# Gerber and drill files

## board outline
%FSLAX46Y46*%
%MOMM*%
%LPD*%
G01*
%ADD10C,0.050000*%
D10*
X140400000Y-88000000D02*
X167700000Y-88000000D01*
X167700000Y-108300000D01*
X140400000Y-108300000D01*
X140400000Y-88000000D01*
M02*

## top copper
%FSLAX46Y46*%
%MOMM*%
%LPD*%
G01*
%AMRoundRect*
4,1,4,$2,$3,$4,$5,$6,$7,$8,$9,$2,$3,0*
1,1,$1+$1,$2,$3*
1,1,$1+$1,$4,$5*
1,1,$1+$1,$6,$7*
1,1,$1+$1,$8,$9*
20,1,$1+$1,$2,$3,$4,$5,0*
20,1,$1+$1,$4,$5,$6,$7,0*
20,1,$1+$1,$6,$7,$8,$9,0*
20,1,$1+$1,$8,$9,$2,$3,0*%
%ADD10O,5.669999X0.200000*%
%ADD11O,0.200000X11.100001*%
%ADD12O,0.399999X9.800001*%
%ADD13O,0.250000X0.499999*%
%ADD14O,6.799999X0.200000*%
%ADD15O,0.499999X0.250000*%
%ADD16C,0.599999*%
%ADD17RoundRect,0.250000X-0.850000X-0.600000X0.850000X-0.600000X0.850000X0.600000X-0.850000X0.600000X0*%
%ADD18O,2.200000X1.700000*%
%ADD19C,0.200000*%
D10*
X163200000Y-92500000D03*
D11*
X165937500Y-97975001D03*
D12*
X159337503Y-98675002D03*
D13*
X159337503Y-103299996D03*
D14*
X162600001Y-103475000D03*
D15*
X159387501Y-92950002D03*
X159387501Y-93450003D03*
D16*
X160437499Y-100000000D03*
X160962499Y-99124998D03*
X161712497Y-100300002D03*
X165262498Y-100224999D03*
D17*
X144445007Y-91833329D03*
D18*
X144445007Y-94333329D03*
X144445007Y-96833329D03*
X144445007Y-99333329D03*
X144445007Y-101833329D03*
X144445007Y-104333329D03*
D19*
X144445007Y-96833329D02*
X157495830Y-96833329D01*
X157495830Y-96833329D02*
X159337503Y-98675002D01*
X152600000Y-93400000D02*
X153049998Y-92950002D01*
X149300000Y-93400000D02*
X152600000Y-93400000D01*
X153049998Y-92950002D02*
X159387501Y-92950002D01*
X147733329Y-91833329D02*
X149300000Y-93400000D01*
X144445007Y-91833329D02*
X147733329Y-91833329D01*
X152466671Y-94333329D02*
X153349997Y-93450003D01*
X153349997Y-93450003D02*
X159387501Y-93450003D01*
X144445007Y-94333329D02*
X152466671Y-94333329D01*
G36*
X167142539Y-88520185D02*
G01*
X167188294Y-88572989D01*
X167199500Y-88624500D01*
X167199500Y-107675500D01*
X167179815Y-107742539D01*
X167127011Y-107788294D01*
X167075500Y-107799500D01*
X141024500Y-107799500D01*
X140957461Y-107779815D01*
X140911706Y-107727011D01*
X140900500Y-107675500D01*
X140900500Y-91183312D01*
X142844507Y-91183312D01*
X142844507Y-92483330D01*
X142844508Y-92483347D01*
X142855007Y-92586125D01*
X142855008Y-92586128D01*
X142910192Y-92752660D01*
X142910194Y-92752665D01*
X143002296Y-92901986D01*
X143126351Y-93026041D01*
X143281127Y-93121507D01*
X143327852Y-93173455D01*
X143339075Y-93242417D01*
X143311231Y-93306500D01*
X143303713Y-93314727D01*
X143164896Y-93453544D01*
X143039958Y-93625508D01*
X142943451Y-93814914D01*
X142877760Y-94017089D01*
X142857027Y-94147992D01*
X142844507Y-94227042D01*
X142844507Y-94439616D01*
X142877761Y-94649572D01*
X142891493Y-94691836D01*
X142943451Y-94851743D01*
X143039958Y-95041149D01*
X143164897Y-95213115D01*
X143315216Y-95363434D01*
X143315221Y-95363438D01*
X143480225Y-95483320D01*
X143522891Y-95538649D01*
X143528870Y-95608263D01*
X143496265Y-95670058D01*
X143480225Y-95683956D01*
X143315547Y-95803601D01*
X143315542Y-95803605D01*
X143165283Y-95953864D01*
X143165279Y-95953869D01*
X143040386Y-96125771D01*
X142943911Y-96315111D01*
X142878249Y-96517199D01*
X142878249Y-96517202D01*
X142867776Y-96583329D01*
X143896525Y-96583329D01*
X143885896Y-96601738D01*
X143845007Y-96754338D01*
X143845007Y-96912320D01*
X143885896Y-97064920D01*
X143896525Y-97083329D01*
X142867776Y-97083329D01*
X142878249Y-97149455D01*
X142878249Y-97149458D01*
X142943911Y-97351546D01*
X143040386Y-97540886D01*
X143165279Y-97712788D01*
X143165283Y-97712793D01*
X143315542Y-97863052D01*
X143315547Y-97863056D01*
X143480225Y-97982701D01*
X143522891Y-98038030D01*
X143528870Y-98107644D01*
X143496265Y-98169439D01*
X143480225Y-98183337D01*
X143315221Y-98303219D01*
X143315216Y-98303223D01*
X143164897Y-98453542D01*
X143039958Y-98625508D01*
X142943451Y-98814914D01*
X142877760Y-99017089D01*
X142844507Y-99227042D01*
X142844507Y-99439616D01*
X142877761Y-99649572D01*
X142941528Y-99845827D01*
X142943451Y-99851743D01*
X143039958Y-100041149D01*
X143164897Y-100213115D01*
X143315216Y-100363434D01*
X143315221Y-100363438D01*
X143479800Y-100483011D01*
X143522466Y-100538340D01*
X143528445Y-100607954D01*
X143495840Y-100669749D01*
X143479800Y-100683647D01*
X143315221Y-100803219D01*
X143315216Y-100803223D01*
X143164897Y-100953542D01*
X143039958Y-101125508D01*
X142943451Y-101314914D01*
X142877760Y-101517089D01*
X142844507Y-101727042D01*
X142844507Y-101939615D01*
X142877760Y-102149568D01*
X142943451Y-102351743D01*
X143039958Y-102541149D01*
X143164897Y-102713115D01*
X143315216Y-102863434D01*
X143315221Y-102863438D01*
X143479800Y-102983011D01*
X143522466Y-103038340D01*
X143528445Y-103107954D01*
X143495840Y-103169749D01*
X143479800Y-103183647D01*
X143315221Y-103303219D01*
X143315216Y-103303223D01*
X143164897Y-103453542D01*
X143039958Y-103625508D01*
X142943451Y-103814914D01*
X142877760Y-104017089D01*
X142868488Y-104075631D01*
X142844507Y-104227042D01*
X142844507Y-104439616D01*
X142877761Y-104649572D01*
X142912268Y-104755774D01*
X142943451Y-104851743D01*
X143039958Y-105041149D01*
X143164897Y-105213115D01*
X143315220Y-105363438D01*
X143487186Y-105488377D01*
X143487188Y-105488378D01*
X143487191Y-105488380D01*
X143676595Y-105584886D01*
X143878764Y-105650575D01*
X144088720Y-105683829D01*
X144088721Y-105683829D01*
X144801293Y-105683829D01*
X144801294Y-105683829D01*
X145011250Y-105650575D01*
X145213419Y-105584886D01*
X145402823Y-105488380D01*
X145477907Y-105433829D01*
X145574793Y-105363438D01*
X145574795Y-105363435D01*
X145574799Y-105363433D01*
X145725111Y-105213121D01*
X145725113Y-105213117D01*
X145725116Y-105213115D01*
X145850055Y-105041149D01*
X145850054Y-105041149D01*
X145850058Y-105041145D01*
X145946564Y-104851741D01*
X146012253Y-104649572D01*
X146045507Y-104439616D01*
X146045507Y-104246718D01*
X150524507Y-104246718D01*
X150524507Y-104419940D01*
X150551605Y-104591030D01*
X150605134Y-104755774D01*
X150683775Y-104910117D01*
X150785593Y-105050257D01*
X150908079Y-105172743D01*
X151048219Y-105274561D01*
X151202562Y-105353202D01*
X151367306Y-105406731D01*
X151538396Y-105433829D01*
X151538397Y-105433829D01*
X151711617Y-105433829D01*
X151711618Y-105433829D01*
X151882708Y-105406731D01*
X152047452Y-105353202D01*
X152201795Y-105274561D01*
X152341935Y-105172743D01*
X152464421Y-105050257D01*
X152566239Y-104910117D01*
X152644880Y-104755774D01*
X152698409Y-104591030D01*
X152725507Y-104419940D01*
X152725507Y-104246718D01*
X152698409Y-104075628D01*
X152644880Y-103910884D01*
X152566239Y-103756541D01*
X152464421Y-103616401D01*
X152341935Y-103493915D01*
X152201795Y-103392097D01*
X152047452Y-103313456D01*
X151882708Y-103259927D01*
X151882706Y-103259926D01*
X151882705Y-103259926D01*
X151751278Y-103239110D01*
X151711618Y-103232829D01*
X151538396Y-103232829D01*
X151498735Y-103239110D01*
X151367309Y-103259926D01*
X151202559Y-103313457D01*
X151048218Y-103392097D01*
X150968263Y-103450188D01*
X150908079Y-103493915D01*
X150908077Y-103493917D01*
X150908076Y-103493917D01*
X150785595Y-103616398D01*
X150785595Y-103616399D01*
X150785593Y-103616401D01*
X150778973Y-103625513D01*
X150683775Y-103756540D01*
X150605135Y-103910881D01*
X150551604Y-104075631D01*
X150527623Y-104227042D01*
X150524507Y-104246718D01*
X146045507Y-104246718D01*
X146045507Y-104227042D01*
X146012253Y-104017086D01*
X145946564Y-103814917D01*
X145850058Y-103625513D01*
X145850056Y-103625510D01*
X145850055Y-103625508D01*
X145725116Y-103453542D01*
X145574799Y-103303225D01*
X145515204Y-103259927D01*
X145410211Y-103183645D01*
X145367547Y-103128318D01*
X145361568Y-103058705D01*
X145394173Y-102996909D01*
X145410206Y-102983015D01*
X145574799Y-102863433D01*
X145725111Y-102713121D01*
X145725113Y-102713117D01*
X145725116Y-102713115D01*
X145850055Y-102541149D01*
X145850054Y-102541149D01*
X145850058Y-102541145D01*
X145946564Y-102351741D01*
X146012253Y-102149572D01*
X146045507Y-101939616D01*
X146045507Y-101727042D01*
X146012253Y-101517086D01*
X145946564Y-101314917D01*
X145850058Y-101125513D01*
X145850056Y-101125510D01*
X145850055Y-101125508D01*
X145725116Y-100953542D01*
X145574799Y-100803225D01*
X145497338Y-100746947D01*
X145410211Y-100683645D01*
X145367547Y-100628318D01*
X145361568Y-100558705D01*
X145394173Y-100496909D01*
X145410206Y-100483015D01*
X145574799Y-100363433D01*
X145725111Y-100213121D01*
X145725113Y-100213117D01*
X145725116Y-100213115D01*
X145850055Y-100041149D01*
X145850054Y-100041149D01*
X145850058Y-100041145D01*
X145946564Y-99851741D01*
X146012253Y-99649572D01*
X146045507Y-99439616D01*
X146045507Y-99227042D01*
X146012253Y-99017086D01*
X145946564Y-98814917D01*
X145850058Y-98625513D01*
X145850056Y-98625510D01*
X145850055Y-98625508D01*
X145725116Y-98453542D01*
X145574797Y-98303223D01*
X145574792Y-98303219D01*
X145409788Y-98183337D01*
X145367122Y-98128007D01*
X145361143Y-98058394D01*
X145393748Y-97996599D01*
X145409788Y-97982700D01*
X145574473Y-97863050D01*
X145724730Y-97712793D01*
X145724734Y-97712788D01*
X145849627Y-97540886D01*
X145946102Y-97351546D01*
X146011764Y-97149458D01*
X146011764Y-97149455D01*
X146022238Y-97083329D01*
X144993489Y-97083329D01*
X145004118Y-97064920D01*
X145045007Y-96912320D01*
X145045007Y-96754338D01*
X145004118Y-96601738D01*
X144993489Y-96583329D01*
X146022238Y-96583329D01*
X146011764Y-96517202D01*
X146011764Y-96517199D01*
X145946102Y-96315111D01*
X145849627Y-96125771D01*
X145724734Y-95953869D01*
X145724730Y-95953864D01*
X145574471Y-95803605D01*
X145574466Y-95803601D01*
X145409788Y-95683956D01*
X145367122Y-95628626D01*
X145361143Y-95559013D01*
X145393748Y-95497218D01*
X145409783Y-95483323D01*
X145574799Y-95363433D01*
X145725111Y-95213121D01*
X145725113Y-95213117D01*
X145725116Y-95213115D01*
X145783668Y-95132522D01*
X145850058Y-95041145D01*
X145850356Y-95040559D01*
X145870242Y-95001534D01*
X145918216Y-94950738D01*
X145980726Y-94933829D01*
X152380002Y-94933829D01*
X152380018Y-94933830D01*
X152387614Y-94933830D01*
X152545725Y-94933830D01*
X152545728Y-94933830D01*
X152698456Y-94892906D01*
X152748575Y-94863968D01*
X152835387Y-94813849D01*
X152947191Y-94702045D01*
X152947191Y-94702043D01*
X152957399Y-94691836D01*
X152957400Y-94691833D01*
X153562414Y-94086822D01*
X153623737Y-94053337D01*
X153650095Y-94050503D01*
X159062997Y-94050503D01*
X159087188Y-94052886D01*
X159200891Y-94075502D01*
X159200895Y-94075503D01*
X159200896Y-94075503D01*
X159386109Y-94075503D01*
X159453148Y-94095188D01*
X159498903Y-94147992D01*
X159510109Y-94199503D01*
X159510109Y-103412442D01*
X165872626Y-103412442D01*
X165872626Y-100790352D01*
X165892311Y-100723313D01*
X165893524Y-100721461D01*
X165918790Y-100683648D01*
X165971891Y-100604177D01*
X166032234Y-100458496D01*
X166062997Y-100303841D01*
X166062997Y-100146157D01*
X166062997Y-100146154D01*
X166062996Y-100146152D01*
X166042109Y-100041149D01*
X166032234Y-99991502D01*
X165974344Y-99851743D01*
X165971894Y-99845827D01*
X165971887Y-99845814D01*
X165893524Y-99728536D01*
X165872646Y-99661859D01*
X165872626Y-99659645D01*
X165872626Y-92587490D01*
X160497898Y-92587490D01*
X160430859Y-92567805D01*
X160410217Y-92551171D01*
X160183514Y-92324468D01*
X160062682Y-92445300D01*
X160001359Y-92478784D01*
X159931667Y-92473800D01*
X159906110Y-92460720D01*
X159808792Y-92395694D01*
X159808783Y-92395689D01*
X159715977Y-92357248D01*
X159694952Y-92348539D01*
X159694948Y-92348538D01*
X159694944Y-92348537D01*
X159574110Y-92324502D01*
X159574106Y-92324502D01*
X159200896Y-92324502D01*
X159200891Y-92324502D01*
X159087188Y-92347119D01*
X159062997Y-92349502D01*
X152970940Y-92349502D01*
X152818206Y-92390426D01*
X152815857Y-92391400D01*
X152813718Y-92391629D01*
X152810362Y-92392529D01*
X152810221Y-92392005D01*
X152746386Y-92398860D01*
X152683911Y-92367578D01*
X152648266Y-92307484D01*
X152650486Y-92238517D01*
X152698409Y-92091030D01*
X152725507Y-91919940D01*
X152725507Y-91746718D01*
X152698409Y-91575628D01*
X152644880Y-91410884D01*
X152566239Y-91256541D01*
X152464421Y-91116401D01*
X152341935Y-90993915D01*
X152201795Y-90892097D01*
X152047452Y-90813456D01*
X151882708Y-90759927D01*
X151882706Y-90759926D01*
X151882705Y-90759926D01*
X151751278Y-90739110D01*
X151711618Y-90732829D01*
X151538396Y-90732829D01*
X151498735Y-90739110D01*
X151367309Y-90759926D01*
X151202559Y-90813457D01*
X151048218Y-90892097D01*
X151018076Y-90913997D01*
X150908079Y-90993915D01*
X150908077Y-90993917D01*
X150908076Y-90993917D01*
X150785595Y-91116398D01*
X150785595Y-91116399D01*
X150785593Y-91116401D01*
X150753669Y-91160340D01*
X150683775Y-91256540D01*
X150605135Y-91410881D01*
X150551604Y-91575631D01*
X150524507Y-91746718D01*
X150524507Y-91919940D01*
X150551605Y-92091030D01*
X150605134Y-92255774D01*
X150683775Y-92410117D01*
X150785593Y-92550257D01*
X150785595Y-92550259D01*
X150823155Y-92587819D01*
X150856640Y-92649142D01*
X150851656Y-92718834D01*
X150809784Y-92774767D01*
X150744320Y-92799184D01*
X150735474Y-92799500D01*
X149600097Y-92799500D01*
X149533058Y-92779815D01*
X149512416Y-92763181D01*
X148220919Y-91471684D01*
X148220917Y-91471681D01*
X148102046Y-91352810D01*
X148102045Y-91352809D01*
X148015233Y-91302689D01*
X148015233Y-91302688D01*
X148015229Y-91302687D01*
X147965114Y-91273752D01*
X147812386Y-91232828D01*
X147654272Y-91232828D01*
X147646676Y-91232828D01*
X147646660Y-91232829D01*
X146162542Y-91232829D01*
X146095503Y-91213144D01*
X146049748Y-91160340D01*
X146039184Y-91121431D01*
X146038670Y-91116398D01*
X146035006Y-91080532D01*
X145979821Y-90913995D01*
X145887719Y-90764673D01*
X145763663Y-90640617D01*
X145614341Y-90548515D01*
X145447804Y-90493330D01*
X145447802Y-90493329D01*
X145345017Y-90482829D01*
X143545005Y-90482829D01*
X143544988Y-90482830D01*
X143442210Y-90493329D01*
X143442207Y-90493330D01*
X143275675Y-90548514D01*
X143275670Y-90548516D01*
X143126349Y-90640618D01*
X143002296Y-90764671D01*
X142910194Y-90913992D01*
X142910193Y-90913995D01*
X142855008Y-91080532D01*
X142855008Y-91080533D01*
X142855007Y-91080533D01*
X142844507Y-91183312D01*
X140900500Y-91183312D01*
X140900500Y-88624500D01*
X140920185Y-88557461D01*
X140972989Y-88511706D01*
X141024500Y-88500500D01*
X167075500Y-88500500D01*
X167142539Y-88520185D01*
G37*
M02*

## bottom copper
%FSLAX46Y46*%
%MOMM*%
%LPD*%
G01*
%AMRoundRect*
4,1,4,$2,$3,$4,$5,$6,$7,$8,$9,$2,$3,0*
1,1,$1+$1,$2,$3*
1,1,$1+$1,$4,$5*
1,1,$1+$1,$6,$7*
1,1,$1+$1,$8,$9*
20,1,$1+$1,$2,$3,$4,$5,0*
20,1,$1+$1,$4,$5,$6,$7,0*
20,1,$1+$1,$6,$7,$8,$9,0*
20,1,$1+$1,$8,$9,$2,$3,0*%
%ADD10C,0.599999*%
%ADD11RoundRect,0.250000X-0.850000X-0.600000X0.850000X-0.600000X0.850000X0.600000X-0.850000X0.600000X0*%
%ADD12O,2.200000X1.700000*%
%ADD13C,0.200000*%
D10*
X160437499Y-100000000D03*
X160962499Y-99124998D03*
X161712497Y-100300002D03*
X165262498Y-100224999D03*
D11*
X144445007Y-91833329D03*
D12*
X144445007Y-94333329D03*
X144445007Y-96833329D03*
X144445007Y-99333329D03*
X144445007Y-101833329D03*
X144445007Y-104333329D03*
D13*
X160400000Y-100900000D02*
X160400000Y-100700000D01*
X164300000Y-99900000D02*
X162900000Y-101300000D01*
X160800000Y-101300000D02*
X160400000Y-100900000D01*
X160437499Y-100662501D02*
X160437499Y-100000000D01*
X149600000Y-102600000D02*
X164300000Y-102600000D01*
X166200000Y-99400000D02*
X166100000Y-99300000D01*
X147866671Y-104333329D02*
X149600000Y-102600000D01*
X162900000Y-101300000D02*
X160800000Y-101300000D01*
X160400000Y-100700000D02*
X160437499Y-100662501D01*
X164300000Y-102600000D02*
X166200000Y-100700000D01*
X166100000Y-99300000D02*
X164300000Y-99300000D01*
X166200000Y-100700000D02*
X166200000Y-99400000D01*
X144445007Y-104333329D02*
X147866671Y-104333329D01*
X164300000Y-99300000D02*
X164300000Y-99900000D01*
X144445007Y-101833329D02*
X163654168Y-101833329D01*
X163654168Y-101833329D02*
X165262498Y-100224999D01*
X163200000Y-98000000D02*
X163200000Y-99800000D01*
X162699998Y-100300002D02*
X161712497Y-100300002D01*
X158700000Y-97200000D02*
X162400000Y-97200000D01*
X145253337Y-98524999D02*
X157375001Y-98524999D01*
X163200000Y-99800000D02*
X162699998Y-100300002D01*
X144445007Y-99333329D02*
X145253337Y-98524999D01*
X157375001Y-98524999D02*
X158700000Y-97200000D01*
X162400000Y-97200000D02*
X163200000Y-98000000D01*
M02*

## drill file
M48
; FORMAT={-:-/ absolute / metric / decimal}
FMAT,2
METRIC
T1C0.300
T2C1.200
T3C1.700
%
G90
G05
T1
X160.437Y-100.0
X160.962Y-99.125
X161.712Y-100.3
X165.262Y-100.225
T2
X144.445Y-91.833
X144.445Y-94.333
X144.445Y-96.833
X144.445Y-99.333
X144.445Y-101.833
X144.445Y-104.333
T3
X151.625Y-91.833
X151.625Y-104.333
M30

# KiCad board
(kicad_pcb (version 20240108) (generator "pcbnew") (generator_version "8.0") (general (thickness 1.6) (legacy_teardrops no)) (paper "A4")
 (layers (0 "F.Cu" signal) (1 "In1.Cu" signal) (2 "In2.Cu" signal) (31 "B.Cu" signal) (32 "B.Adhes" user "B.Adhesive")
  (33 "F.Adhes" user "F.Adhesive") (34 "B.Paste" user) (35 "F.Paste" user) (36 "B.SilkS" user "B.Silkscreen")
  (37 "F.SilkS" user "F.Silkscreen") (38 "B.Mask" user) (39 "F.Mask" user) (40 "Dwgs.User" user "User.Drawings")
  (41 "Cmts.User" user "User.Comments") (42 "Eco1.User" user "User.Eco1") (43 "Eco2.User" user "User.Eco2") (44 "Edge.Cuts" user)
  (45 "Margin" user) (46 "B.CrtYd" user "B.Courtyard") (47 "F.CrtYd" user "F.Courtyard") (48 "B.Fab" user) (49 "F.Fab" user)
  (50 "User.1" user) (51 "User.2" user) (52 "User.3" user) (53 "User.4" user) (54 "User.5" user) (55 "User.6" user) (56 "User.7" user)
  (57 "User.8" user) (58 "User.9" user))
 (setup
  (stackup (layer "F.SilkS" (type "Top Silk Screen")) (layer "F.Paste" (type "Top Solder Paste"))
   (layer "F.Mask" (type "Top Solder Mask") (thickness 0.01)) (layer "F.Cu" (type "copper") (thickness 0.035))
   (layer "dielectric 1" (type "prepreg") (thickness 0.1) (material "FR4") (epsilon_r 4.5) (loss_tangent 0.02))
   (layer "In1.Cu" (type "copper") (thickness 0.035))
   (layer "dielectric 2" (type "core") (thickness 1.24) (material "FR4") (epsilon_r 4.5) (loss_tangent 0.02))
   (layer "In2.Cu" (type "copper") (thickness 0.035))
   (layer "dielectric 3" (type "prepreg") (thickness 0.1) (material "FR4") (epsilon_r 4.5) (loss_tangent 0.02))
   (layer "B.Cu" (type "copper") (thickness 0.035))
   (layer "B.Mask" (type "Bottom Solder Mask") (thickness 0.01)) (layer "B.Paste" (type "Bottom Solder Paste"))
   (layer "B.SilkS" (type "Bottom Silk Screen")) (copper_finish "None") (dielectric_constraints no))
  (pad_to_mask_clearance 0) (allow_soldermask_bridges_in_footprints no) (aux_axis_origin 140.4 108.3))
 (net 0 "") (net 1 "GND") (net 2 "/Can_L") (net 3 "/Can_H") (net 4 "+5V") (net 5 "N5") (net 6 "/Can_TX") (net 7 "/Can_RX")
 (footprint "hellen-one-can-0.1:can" (layer "F.Cu") (at 159.0625 92.300003 -90)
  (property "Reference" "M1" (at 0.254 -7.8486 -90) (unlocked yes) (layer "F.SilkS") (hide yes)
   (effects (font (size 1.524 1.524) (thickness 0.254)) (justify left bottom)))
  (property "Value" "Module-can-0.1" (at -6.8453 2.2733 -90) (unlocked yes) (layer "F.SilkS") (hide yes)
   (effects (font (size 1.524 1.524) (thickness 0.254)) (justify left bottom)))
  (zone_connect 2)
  (pad "E1" smd oval (at 0.199997 -4.1375 90) (size 0.2 5.669999) (layers "F.Cu" "F.Paste") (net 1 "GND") (solder_mask_margin 0.1016)
   (solder_paste_margin -49.999999) (zone_connect 2))
  (pad "E1" smd oval (at 5.674998 -6.875) (size 0.2 11.100001) (layers "F.Cu" "F.Paste") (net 1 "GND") (solder_mask_margin 0.1016)
   (solder_paste_margin -49.999999) (zone_connect 2))
  (pad "E1" smd oval (at 6.374999 -0.275003 180) (size 0.399999 9.800001) (layers "F.Cu" "F.Paste") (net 1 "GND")
   (solder_mask_margin 0.1016) (solder_paste_margin -49.999999) (zone_connect 2))
  (pad "E1" smd oval (at 10.999993 -0.275003 90) (size 0.499999 0.25) (layers "F.Cu" "F.Paste" "F.Mask") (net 1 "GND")
   (solder_paste_margin -49.999999) (zone_connect 2))
  (pad "E1" smd oval (at 11.174997 -3.537501 90) (size 0.2 6.799999) (layers "F.Cu" "F.Paste") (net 1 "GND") (solder_mask_margin 0.1016)
   (solder_paste_margin -49.999999) (zone_connect 2))
  (pad "S1" smd oval (at 0.649999 -0.325001 270) (size 0.25 0.499999) (layers "F.Cu" "F.Paste" "F.Mask") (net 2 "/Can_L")
   (solder_paste_margin -49.999999) (zone_connect 2))
  (pad "S2" smd oval (at 1.15 -0.325001 270) (size 0.25 0.499999) (layers "F.Cu" "F.Paste" "F.Mask") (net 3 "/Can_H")
   (solder_paste_margin -49.999999) (zone_connect 2))
  (pad "V1" thru_hole circle (at 7.699997 -1.374999 90) (size 0.599999 0.599999) (drill 0.299999) (layers "*.Cu" "*.Mask")
   (remove_unused_layers no) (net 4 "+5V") (solder_paste_margin -49.999999) (zone_connect 2))
  (pad "V2" thru_hole circle (at 6.824995 -1.899999 90) (size 0.599999 0.599999) (drill 0.299999) (layers "*.Cu" "*.Mask")
   (remove_unused_layers no) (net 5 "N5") (solder_paste_margin -49.999999) (zone_connect 2))
  (pad "V5" thru_hole circle (at 7.999999 -2.649997 180) (size 0.599999 0.599999) (drill 0.299999) (layers "*.Cu" "*.Mask")
   (remove_unused_layers no) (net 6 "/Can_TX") (solder_paste_margin -49.999999) (zone_connect 2))
  (pad "V6" thru_hole circle (at 7.924996 -6.199998 180) (size 0.599999 0.599999) (drill 0.299999) (layers "*.Cu" "*.Mask")
   (remove_unused_layers no) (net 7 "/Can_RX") (solder_paste_margin -49.999999) (zone_connect 2))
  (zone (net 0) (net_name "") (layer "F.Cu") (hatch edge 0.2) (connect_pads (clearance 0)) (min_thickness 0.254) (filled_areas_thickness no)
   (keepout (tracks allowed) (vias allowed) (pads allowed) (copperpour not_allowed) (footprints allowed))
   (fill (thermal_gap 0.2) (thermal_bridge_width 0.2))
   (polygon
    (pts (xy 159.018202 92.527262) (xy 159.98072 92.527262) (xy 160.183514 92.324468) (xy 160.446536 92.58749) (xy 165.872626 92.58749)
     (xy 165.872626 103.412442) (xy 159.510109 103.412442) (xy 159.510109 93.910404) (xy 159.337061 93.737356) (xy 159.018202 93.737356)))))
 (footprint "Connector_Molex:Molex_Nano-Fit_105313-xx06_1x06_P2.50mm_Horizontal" (layer "F.Cu") (at 144.445007 91.833329)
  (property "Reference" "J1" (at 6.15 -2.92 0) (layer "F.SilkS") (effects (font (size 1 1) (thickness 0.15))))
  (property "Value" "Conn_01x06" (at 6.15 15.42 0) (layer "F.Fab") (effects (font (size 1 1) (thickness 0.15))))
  (pad "" np_thru_hole circle (at 7.18 0) (size 1.7 1.7) (drill 1.7) (layers "*.Cu" "*.Mask"))
  (pad "" np_thru_hole circle (at 7.18 12.5) (size 1.7 1.7) (drill 1.7) (layers "*.Cu" "*.Mask"))
  (pad "1" thru_hole roundrect (at 0 0) (size 2.2 1.7) (drill 1.2) (layers "*.Cu" "*.Mask") (remove_unused_layers no)
   (roundrect_rratio 0.147059) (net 2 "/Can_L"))
  (pad "2" thru_hole oval (at 0 2.5) (size 2.2 1.7) (drill 1.2) (layers "*.Cu" "*.Mask") (remove_unused_layers no) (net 3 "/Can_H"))
  (pad "3" thru_hole oval (at 0 5) (size 2.2 1.7) (drill 1.2) (layers "*.Cu" "*.Mask") (remove_unused_layers no) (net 1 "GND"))
  (pad "4" thru_hole oval (at 0 7.5) (size 2.2 1.7) (drill 1.2) (layers "*.Cu" "*.Mask") (remove_unused_layers no) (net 6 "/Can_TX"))
  (pad "5" thru_hole oval (at 0 10) (size 2.2 1.7) (drill 1.2) (layers "*.Cu" "*.Mask") (remove_unused_layers no) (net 7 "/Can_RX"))
  (pad "6" thru_hole oval (at 0 12.5) (size 2.2 1.7) (drill 1.2) (layers "*.Cu" "*.Mask") (remove_unused_layers no) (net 4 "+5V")))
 (gr_rect (start 140.4 88) (end 167.7 108.3) (stroke (width 0.05) (type default)) (fill none) (layer "Edge.Cuts"))
 (segment (start 144.445007 96.833329) (end 157.49583 96.833329) (width 0.2) (layer "F.Cu") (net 1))
 (segment (start 157.49583 96.833329) (end 159.337503 98.675002) (width 0.2) (layer "F.Cu") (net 1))
 (segment (start 160.4 100.9) (end 160.4 100.7) (width 0.2) (layer "B.Cu") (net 4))
 (segment (start 164.3 99.9) (end 162.9 101.3) (width 0.2) (layer "B.Cu") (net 4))
 (segment (start 160.8 101.3) (end 160.4 100.9) (width 0.2) (layer "B.Cu") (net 4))
 (segment (start 160.437499 100.662501) (end 160.437499 100) (width 0.2) (layer "B.Cu") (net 4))
 (segment (start 149.6 102.6) (end 164.3 102.6) (width 0.2) (layer "B.Cu") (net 4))
 (segment (start 166.2 99.4) (end 166.1 99.3) (width 0.2) (layer "B.Cu") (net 4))
 (segment (start 147.866671 104.333329) (end 149.6 102.6) (width 0.2) (layer "B.Cu") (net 4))
 (segment (start 162.9 101.3) (end 160.8 101.3) (width 0.2) (layer "B.Cu") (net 4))
 (segment (start 160.4 100.7) (end 160.437499 100.662501) (width 0.2) (layer "B.Cu") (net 4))
 (segment (start 164.3 102.6) (end 166.2 100.7) (width 0.2) (layer "B.Cu") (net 4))
 (segment (start 166.1 99.3) (end 164.3 99.3) (width 0.2) (layer "B.Cu") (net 4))
 (segment (start 166.2 100.7) (end 166.2 99.4) (width 0.2) (layer "B.Cu") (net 4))
 (segment (start 144.445007 104.333329) (end 147.866671 104.333329) (width 0.2) (layer "B.Cu") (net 4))
 (segment (start 164.3 99.3) (end 164.3 99.9) (width 0.2) (layer "B.Cu") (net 4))
 (segment (start 152.6 93.4) (end 153.049998 92.950002) (width 0.2) (layer "F.Cu") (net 2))
 (segment (start 149.3 93.4) (end 152.6 93.4) (width 0.2) (layer "F.Cu") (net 2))
 (segment (start 153.049998 92.950002) (end 159.387501 92.950002) (width 0.2) (layer "F.Cu") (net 2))
 (segment (start 147.733329 91.833329) (end 149.3 93.4) (width 0.2) (layer "F.Cu") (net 2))
 (segment (start 144.445007 91.833329) (end 147.733329 91.833329) (width 0.2) (layer "F.Cu") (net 2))
 (segment (start 152.466671 94.333329) (end 153.349997 93.450003) (width 0.2) (layer "F.Cu") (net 3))
 (segment (start 153.349997 93.450003) (end 159.387501 93.450003) (width 0.2) (layer "F.Cu") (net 3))
 (segment (start 144.445007 94.333329) (end 152.466671 94.333329) (width 0.2) (layer "F.Cu") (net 3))
 (segment (start 144.445007 101.833329) (end 163.654168 101.833329) (width 0.2) (layer "B.Cu") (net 7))
 (segment (start 163.654168 101.833329) (end 165.262498 100.224999) (width 0.2) (layer "B.Cu") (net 7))
 (segment (start 163.2 98) (end 163.2 99.8) (width 0.2) (layer "B.Cu") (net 6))
 (segment (start 162.699998 100.300002) (end 161.712497 100.300002) (width 0.2) (layer "B.Cu") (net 6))
 (segment (start 158.7 97.2) (end 162.4 97.2) (width 0.2) (layer "B.Cu") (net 6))
 (segment (start 145.253337 98.524999) (end 157.375001 98.524999) (width 0.2) (layer "B.Cu") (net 6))
 (segment (start 163.2 99.8) (end 162.699998 100.300002) (width 0.2) (layer "B.Cu") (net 6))
 (segment (start 144.445007 99.333329) (end 145.253337 98.524999) (width 0.2) (layer "B.Cu") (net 6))
 (segment (start 157.375001 98.524999) (end 158.7 97.2) (width 0.2) (layer "B.Cu") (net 6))
 (segment (start 162.4 97.2) (end 163.2 98) (width 0.2) (layer "B.Cu") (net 6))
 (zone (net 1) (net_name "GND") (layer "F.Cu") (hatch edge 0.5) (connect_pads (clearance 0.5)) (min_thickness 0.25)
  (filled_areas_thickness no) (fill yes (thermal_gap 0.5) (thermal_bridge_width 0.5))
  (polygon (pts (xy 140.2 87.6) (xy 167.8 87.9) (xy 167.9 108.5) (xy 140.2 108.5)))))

